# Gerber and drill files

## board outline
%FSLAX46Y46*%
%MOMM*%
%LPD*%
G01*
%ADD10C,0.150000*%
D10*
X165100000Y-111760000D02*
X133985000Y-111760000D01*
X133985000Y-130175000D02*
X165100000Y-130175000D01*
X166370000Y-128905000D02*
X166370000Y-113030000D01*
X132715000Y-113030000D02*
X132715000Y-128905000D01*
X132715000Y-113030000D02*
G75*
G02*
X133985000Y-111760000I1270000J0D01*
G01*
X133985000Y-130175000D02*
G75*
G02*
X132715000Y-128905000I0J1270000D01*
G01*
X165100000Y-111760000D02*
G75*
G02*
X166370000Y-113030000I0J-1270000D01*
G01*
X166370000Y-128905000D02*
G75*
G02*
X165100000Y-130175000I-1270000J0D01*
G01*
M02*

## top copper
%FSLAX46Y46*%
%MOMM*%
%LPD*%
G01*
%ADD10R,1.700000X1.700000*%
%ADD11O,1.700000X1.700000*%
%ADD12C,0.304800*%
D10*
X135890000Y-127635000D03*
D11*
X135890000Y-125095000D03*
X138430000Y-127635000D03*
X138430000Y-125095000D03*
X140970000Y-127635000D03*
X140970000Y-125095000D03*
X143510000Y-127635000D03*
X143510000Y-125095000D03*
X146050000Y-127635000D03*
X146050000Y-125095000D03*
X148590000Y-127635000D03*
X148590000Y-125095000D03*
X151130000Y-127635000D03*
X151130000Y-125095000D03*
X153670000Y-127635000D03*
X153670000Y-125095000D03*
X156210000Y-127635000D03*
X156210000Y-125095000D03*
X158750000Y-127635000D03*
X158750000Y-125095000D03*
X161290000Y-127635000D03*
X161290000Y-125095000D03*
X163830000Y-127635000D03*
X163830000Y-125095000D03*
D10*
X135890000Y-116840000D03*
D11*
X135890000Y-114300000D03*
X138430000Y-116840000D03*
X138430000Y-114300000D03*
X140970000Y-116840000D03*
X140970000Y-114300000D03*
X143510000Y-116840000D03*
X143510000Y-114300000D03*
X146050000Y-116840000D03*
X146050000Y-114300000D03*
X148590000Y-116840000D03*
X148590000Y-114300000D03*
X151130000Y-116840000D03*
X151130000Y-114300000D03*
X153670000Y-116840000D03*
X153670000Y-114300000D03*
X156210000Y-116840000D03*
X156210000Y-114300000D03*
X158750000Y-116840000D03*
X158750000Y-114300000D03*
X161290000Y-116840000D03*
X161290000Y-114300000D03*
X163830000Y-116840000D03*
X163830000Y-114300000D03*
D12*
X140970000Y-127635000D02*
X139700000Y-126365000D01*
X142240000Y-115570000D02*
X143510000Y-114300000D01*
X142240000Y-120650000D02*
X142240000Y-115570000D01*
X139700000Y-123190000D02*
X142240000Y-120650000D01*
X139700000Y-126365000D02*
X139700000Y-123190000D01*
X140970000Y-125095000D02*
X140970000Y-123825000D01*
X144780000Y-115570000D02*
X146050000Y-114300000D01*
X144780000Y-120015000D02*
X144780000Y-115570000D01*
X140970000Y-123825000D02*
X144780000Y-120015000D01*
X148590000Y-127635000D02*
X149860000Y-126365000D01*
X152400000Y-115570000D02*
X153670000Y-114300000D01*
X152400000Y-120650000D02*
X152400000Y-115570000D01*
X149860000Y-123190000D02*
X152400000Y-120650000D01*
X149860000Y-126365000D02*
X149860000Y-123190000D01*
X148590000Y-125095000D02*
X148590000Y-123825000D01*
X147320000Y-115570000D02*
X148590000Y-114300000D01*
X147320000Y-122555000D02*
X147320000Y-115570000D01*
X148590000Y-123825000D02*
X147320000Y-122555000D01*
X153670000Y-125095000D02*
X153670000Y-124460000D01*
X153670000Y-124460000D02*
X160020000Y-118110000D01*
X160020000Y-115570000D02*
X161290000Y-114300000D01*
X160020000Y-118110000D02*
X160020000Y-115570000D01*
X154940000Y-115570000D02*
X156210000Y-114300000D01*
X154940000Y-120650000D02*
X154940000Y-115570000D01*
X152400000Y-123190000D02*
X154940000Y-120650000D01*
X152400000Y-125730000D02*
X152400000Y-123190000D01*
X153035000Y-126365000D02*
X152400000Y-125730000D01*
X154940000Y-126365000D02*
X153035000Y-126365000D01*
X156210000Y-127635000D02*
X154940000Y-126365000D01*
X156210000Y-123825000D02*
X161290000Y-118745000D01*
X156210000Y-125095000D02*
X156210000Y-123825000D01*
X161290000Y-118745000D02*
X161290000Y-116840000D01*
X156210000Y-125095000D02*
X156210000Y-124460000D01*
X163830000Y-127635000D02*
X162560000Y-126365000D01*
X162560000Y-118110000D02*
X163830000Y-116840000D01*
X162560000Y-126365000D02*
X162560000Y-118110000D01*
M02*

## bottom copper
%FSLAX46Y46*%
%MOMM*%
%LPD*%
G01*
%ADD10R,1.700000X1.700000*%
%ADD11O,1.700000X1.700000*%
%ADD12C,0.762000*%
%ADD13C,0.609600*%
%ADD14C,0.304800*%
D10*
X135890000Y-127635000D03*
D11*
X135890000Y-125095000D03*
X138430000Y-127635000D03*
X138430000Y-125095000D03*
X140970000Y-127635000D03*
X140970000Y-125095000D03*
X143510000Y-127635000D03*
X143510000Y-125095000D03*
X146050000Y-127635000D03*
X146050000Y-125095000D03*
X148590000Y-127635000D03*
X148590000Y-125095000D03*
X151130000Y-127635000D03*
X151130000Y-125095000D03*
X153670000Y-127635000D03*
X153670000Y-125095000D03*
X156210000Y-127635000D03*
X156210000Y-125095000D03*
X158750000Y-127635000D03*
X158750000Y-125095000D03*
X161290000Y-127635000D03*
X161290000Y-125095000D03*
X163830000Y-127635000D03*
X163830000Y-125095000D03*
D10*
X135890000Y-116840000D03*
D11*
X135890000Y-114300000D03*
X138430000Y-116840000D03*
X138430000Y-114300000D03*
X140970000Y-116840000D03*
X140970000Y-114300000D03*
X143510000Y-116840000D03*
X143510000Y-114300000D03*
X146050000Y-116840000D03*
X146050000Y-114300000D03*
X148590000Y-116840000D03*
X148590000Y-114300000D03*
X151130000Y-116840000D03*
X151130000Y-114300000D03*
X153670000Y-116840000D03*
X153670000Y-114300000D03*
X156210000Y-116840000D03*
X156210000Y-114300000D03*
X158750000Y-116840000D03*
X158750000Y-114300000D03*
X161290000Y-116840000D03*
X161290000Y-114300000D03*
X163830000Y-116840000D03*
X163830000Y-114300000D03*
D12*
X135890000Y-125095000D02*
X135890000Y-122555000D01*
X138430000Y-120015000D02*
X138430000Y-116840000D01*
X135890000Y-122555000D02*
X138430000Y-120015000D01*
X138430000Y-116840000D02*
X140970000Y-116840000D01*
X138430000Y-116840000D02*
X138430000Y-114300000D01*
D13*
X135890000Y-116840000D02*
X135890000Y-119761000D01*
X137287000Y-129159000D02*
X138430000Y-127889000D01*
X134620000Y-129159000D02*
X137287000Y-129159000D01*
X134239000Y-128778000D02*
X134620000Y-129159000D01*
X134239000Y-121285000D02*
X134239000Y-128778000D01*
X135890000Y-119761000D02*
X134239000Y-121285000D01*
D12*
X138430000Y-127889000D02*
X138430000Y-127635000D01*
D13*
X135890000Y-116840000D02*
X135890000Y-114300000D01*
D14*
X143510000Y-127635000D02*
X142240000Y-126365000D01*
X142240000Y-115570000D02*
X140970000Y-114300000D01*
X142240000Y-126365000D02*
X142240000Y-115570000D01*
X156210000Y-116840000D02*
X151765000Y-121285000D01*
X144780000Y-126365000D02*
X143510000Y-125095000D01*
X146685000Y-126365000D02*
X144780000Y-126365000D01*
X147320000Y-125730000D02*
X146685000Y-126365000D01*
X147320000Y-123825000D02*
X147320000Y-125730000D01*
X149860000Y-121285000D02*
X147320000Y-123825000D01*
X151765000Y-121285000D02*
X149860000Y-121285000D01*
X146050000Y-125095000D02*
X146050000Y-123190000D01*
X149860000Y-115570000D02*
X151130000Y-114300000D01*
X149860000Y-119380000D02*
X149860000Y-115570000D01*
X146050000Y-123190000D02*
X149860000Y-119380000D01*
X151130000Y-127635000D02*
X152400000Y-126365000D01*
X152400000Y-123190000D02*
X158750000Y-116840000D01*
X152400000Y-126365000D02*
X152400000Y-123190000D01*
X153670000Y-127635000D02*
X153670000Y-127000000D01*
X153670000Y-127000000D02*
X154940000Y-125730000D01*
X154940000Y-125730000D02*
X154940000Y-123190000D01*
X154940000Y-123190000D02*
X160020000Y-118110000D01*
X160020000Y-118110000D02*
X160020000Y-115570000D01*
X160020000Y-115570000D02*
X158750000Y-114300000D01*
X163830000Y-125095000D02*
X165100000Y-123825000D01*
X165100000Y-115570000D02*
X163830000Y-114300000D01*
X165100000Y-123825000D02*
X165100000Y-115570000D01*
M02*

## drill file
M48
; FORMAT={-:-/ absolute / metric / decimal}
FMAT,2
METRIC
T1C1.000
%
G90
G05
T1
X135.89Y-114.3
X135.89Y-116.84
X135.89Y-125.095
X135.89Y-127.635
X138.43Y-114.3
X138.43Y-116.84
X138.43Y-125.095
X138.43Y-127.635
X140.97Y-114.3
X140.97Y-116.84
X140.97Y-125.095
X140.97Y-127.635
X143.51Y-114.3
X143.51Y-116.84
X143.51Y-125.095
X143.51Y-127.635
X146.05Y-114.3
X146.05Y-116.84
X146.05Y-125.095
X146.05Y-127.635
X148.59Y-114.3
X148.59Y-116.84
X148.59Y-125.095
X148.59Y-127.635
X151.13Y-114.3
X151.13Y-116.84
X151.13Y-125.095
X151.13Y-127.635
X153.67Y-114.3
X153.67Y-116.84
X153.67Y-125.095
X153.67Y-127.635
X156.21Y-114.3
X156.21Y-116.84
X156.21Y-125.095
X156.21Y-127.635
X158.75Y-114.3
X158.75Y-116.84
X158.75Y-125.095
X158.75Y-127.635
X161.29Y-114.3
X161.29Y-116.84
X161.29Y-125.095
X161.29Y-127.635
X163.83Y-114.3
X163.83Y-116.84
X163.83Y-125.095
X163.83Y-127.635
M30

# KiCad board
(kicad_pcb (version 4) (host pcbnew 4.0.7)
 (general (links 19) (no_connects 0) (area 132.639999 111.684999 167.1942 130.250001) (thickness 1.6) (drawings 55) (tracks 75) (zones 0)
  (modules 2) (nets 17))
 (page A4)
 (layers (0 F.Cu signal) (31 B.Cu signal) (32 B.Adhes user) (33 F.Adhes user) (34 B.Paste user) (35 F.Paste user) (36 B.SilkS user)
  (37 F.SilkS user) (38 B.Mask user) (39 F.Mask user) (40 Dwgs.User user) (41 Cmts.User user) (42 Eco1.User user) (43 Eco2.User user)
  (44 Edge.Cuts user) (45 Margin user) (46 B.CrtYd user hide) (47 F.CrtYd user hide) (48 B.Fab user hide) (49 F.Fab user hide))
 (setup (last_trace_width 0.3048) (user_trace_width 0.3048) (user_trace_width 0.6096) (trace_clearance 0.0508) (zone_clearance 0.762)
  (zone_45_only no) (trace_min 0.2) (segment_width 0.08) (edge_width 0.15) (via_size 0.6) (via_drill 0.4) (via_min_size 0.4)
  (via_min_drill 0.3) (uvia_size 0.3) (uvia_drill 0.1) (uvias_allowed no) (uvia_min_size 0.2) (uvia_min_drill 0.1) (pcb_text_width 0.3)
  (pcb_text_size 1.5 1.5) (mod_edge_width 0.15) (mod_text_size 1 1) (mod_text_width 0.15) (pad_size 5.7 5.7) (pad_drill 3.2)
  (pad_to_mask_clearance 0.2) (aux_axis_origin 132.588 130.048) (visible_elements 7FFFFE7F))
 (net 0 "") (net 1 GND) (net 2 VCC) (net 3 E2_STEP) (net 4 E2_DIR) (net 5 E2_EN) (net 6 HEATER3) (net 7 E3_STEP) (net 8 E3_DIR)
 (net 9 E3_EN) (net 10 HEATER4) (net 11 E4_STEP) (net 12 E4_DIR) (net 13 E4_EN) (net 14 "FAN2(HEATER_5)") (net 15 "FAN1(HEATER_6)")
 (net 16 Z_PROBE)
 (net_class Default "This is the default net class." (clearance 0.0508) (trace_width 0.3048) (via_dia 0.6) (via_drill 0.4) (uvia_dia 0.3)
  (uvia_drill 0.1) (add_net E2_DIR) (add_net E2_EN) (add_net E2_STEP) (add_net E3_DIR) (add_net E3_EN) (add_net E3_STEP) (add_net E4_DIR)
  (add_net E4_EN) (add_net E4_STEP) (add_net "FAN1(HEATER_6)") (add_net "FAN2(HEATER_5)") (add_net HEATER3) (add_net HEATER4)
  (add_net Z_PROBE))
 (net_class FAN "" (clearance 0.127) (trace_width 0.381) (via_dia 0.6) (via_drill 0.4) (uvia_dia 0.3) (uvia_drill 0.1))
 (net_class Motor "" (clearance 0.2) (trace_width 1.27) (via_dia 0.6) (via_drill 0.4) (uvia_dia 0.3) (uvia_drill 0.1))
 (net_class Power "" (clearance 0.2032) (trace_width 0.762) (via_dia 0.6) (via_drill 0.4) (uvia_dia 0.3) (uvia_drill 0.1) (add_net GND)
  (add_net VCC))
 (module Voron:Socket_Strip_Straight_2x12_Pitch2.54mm (layer B.Cu) (at 135.89 127.635 270)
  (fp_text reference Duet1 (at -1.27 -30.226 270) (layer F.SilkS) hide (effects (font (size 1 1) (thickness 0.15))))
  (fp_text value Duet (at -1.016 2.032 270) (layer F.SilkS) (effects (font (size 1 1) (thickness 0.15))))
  (pad 1 thru_hole rect (at 0 0 270) (size 1.7 1.7) (drill 1) (layers *.Cu *.Mask))
  (pad 2 thru_hole oval (at -2.54 0 270) (size 1.7 1.7) (drill 1) (layers *.Cu *.Mask) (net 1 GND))
  (pad 3 thru_hole oval (at 0 -2.54 270) (size 1.7 1.7) (drill 1) (layers *.Cu *.Mask) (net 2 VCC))
  (pad 4 thru_hole oval (at -2.54 -2.54 270) (size 1.7 1.7) (drill 1) (layers *.Cu *.Mask))
  (pad 5 thru_hole oval (at 0 -5.08 270) (size 1.7 1.7) (drill 1) (layers *.Cu *.Mask) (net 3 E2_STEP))
  (pad 6 thru_hole oval (at -2.54 -5.08 270) (size 1.7 1.7) (drill 1) (layers *.Cu *.Mask) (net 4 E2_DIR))
  (pad 7 thru_hole oval (at 0 -7.62 270) (size 1.7 1.7) (drill 1) (layers *.Cu *.Mask) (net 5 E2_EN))
  (pad 8 thru_hole oval (at -2.54 -7.62 270) (size 1.7 1.7) (drill 1) (layers *.Cu *.Mask) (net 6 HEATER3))
  (pad 9 thru_hole oval (at 0 -10.16 270) (size 1.7 1.7) (drill 1) (layers *.Cu *.Mask))
  (pad 10 thru_hole oval (at -2.54 -10.16 270) (size 1.7 1.7) (drill 1) (layers *.Cu *.Mask) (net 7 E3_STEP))
  (pad 11 thru_hole oval (at 0 -12.7 270) (size 1.7 1.7) (drill 1) (layers *.Cu *.Mask) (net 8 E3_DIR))
  (pad 12 thru_hole oval (at -2.54 -12.7 270) (size 1.7 1.7) (drill 1) (layers *.Cu *.Mask) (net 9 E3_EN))
  (pad 13 thru_hole oval (at 0 -15.24 270) (size 1.7 1.7) (drill 1) (layers *.Cu *.Mask) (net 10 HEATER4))
  (pad 14 thru_hole oval (at -2.54 -15.24 270) (size 1.7 1.7) (drill 1) (layers *.Cu *.Mask))
  (pad 15 thru_hole oval (at 0 -17.78 270) (size 1.7 1.7) (drill 1) (layers *.Cu *.Mask) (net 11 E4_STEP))
  (pad 16 thru_hole oval (at -2.54 -17.78 270) (size 1.7 1.7) (drill 1) (layers *.Cu *.Mask) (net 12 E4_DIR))
  (pad 17 thru_hole oval (at 0 -20.32 270) (size 1.7 1.7) (drill 1) (layers *.Cu *.Mask) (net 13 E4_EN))
  (pad 18 thru_hole oval (at -2.54 -20.32 270) (size 1.7 1.7) (drill 1) (layers *.Cu *.Mask) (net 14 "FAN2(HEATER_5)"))
  (pad 19 thru_hole oval (at 0 -22.86 270) (size 1.7 1.7) (drill 1) (layers *.Cu *.Mask))
  (pad 20 thru_hole oval (at -2.54 -22.86 270) (size 1.7 1.7) (drill 1) (layers *.Cu *.Mask))
  (pad 21 thru_hole oval (at 0 -25.4 270) (size 1.7 1.7) (drill 1) (layers *.Cu *.Mask))
  (pad 22 thru_hole oval (at -2.54 -25.4 270) (size 1.7 1.7) (drill 1) (layers *.Cu *.Mask))
  (pad 23 thru_hole oval (at 0 -27.94 270) (size 1.7 1.7) (drill 1) (layers *.Cu *.Mask) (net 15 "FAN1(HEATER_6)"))
  (pad 24 thru_hole oval (at -2.54 -27.94 270) (size 1.7 1.7) (drill 1) (layers *.Cu *.Mask) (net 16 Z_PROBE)))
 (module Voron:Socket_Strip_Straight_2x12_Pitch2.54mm (layer B.Cu) (at 135.89 116.84 270)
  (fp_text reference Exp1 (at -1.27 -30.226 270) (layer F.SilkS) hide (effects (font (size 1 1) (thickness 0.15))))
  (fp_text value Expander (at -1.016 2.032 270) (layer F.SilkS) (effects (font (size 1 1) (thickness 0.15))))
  (pad 1 thru_hole rect (at 0 0 270) (size 1.7 1.7) (drill 1) (layers *.Cu *.Mask) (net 2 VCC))
  (pad 2 thru_hole oval (at -2.54 0 270) (size 1.7 1.7) (drill 1) (layers *.Cu *.Mask) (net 2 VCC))
  (pad 3 thru_hole oval (at 0 -2.54 270) (size 1.7 1.7) (drill 1) (layers *.Cu *.Mask) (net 1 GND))
  (pad 4 thru_hole oval (at -2.54 -2.54 270) (size 1.7 1.7) (drill 1) (layers *.Cu *.Mask) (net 1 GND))
  (pad 5 thru_hole oval (at 0 -5.08 270) (size 1.7 1.7) (drill 1) (layers *.Cu *.Mask) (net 1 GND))
  (pad 6 thru_hole oval (at -2.54 -5.08 270) (size 1.7 1.7) (drill 1) (layers *.Cu *.Mask) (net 5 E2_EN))
  (pad 7 thru_hole oval (at 0 -7.62 270) (size 1.7 1.7) (drill 1) (layers *.Cu *.Mask))
  (pad 8 thru_hole oval (at -2.54 -7.62 270) (size 1.7 1.7) (drill 1) (layers *.Cu *.Mask) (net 3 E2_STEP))
  (pad 9 thru_hole oval (at 0 -10.16 270) (size 1.7 1.7) (drill 1) (layers *.Cu *.Mask))
  (pad 10 thru_hole oval (at -2.54 -10.16 270) (size 1.7 1.7) (drill 1) (layers *.Cu *.Mask) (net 4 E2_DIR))
  (pad 11 thru_hole oval (at 0 -12.7 270) (size 1.7 1.7) (drill 1) (layers *.Cu *.Mask))
  (pad 12 thru_hole oval (at -2.54 -12.7 270) (size 1.7 1.7) (drill 1) (layers *.Cu *.Mask) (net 9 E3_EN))
  (pad 13 thru_hole oval (at 0 -15.24 270) (size 1.7 1.7) (drill 1) (layers *.Cu *.Mask))
  (pad 14 thru_hole oval (at -2.54 -15.24 270) (size 1.7 1.7) (drill 1) (layers *.Cu *.Mask) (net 7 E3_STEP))
  (pad 15 thru_hole oval (at 0 -17.78 270) (size 1.7 1.7) (drill 1) (layers *.Cu *.Mask))
  (pad 16 thru_hole oval (at -2.54 -17.78 270) (size 1.7 1.7) (drill 1) (layers *.Cu *.Mask) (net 8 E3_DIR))
  (pad 17 thru_hole oval (at 0 -20.32 270) (size 1.7 1.7) (drill 1) (layers *.Cu *.Mask) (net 6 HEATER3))
  (pad 18 thru_hole oval (at -2.54 -20.32 270) (size 1.7 1.7) (drill 1) (layers *.Cu *.Mask) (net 13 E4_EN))
  (pad 19 thru_hole oval (at 0 -22.86 270) (size 1.7 1.7) (drill 1) (layers *.Cu *.Mask) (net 10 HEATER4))
  (pad 20 thru_hole oval (at -2.54 -22.86 270) (size 1.7 1.7) (drill 1) (layers *.Cu *.Mask) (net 11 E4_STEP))
  (pad 21 thru_hole oval (at 0 -25.4 270) (size 1.7 1.7) (drill 1) (layers *.Cu *.Mask) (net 14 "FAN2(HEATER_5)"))
  (pad 22 thru_hole oval (at -2.54 -25.4 270) (size 1.7 1.7) (drill 1) (layers *.Cu *.Mask) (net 12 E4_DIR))
  (pad 23 thru_hole oval (at 0 -27.94 270) (size 1.7 1.7) (drill 1) (layers *.Cu *.Mask) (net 15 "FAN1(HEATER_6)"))
  (pad 24 thru_hole oval (at -2.54 -27.94 270) (size 1.7 1.7) (drill 1) (layers *.Cu *.Mask) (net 16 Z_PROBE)))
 (gr_line (start 165.1 111.76) (end 133.985 111.76) (angle 90) (layer Edge.Cuts) (width 0.15))
 (gr_line (start 133.985 130.175) (end 165.1 130.175) (angle 90) (layer Edge.Cuts) (width 0.15))
 (gr_line (start 166.37 128.905) (end 166.37 113.03) (angle 90) (layer Edge.Cuts) (width 0.15))
 (gr_line (start 132.715 113.03) (end 132.715 128.905) (angle 90) (layer Edge.Cuts) (width 0.15))
 (gr_arc (start 133.985 113.03) (end 132.715 113.03) (angle 90) (layer Edge.Cuts) (width 0.15))
 (gr_arc (start 133.985 128.905) (end 133.985 130.175) (angle 90) (layer Edge.Cuts) (width 0.15))
 (gr_arc (start 165.1 113.03) (end 165.1 111.76) (angle 90) (layer Edge.Cuts) (width 0.15))
 (gr_arc (start 165.1 128.905) (end 166.37 128.905) (angle 90) (layer Edge.Cuts) (width 0.15))
 (segment (start 135.89 125.095) (end 135.89 122.555) (width 0.762) (layer B.Cu) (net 1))
 (segment (start 138.43 120.015) (end 138.43 116.84) (width 0.762) (layer B.Cu) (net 1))
 (segment (start 135.89 122.555) (end 138.43 120.015) (width 0.762) (layer B.Cu) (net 1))
 (segment (start 138.43 116.84) (end 140.97 116.84) (width 0.762) (layer B.Cu) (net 1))
 (segment (start 138.43 116.84) (end 138.43 114.3) (width 0.762) (layer B.Cu) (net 1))
 (segment (start 135.89 116.84) (end 135.89 119.761) (width 0.6096) (layer B.Cu) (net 2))
 (segment (start 137.287 129.159) (end 138.43 127.889) (width 0.6096) (layer B.Cu) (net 2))
 (segment (start 134.62 129.159) (end 137.287 129.159) (width 0.6096) (layer B.Cu) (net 2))
 (segment (start 134.239 128.778) (end 134.62 129.159) (width 0.6096) (layer B.Cu) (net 2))
 (segment (start 134.239 121.285) (end 134.239 128.778) (width 0.6096) (layer B.Cu) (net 2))
 (segment (start 135.89 119.761) (end 134.239 121.285) (width 0.6096) (layer B.Cu) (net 2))
 (segment (start 138.43 127.889) (end 138.43 127.635) (width 0.762) (layer B.Cu) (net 2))
 (segment (start 135.89 116.84) (end 135.89 114.3) (width 0.6096) (layer B.Cu) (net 2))
 (segment (start 140.97 127.635) (end 139.7 126.365) (width 0.3048) (layer F.Cu) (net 3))
 (segment (start 142.24 115.57) (end 143.51 114.3) (width 0.3048) (layer F.Cu) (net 3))
 (segment (start 142.24 120.65) (end 142.24 115.57) (width 0.3048) (layer F.Cu) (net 3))
 (segment (start 139.7 123.19) (end 142.24 120.65) (width 0.3048) (layer F.Cu) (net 3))
 (segment (start 139.7 126.365) (end 139.7 123.19) (width 0.3048) (layer F.Cu) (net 3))
 (segment (start 140.97 125.095) (end 140.97 123.825) (width 0.3048) (layer F.Cu) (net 4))
 (segment (start 144.78 115.57) (end 146.05 114.3) (width 0.3048) (layer F.Cu) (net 4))
 (segment (start 144.78 120.015) (end 144.78 115.57) (width 0.3048) (layer F.Cu) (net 4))
 (segment (start 140.97 123.825) (end 144.78 120.015) (width 0.3048) (layer F.Cu) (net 4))
 (segment (start 143.51 127.635) (end 142.24 126.365) (width 0.3048) (layer B.Cu) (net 5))
 (segment (start 142.24 115.57) (end 140.97 114.3) (width 0.3048) (layer B.Cu) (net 5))
 (segment (start 142.24 126.365) (end 142.24 115.57) (width 0.3048) (layer B.Cu) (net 5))
 (segment (start 156.21 116.84) (end 151.765 121.285) (width 0.3048) (layer B.Cu) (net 6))
 (segment (start 144.78 126.365) (end 143.51 125.095) (width 0.3048) (layer B.Cu) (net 6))
 (segment (start 146.685 126.365) (end 144.78 126.365) (width 0.3048) (layer B.Cu) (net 6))
 (segment (start 147.32 125.73) (end 146.685 126.365) (width 0.3048) (layer B.Cu) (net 6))
 (segment (start 147.32 123.825) (end 147.32 125.73) (width 0.3048) (layer B.Cu) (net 6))
 (segment (start 149.86 121.285) (end 147.32 123.825) (width 0.3048) (layer B.Cu) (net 6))
 (segment (start 151.765 121.285) (end 149.86 121.285) (width 0.3048) (layer B.Cu) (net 6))
 (segment (start 146.05 125.095) (end 146.05 123.19) (width 0.3048) (layer B.Cu) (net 7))
 (segment (start 149.86 115.57) (end 151.13 114.3) (width 0.3048) (layer B.Cu) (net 7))
 (segment (start 149.86 119.38) (end 149.86 115.57) (width 0.3048) (layer B.Cu) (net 7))
 (segment (start 146.05 123.19) (end 149.86 119.38) (width 0.3048) (layer B.Cu) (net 7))
 (segment (start 148.59 127.635) (end 149.86 126.365) (width 0.3048) (layer F.Cu) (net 8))
 (segment (start 152.4 115.57) (end 153.67 114.3) (width 0.3048) (layer F.Cu) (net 8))
 (segment (start 152.4 120.65) (end 152.4 115.57) (width 0.3048) (layer F.Cu) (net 8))
 (segment (start 149.86 123.19) (end 152.4 120.65) (width 0.3048) (layer F.Cu) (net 8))
 (segment (start 149.86 126.365) (end 149.86 123.19) (width 0.3048) (layer F.Cu) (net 8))
 (segment (start 148.59 125.095) (end 148.59 123.825) (width 0.3048) (layer F.Cu) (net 9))
 (segment (start 147.32 115.57) (end 148.59 114.3) (width 0.3048) (layer F.Cu) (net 9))
 (segment (start 147.32 122.555) (end 147.32 115.57) (width 0.3048) (layer F.Cu) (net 9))
 (segment (start 148.59 123.825) (end 147.32 122.555) (width 0.3048) (layer F.Cu) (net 9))
 (segment (start 151.13 127.635) (end 152.4 126.365) (width 0.3048) (layer B.Cu) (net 10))
 (segment (start 152.4 123.19) (end 158.75 116.84) (width 0.3048) (layer B.Cu) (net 10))
 (segment (start 152.4 126.365) (end 152.4 123.19) (width 0.3048) (layer B.Cu) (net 10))
 (segment (start 153.67 127.635) (end 153.67 127) (width 0.3048) (layer B.Cu) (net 11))
 (segment (start 153.67 127) (end 154.94 125.73) (width 0.3048) (layer B.Cu) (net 11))
 (segment (start 154.94 125.73) (end 154.94 123.19) (width 0.3048) (layer B.Cu) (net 11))
 (segment (start 154.94 123.19) (end 160.02 118.11) (width 0.3048) (layer B.Cu) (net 11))
 (segment (start 160.02 118.11) (end 160.02 115.57) (width 0.3048) (layer B.Cu) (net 11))
 (segment (start 160.02 115.57) (end 158.75 114.3) (width 0.3048) (layer B.Cu) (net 11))
 (segment (start 153.67 125.095) (end 153.67 124.46) (width 0.3048) (layer F.Cu) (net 12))
 (segment (start 153.67 124.46) (end 160.02 118.11) (width 0.3048) (layer F.Cu) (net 12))
 (segment (start 160.02 115.57) (end 161.29 114.3) (width 0.3048) (layer F.Cu) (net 12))
 (segment (start 160.02 118.11) (end 160.02 115.57) (width 0.3048) (layer F.Cu) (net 12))
 (segment (start 154.94 115.57) (end 156.21 114.3) (width 0.3048) (layer F.Cu) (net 13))
 (segment (start 154.94 120.65) (end 154.94 115.57) (width 0.3048) (layer F.Cu) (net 13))
 (segment (start 152.4 123.19) (end 154.94 120.65) (width 0.3048) (layer F.Cu) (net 13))
 (segment (start 152.4 125.73) (end 152.4 123.19) (width 0.3048) (layer F.Cu) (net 13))
 (segment (start 153.035 126.365) (end 152.4 125.73) (width 0.3048) (layer F.Cu) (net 13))
 (segment (start 154.94 126.365) (end 153.035 126.365) (width 0.3048) (layer F.Cu) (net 13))
 (segment (start 156.21 127.635) (end 154.94 126.365) (width 0.3048) (layer F.Cu) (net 13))
 (segment (start 156.21 123.825) (end 161.29 118.745) (width 0.3048) (layer F.Cu) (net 14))
 (segment (start 156.21 125.095) (end 156.21 123.825) (width 0.3048) (layer F.Cu) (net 14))
 (segment (start 161.29 118.745) (end 161.29 116.84) (width 0.3048) (layer F.Cu) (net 14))
 (segment (start 156.21 125.095) (end 156.21 124.46) (width 0.3048) (layer F.Cu) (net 14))
 (segment (start 163.83 127.635) (end 162.56 126.365) (width 0.3048) (layer F.Cu) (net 15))
 (segment (start 162.56 118.11) (end 163.83 116.84) (width 0.3048) (layer F.Cu) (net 15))
 (segment (start 162.56 126.365) (end 162.56 118.11) (width 0.3048) (layer F.Cu) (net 15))
 (segment (start 163.83 125.095) (end 165.1 123.825) (width 0.3048) (layer B.Cu) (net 16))
 (segment (start 165.1 115.57) (end 163.83 114.3) (width 0.3048) (layer B.Cu) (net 16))
 (segment (start 165.1 123.825) (end 165.1 115.57) (width 0.3048) (layer B.Cu) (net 16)))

